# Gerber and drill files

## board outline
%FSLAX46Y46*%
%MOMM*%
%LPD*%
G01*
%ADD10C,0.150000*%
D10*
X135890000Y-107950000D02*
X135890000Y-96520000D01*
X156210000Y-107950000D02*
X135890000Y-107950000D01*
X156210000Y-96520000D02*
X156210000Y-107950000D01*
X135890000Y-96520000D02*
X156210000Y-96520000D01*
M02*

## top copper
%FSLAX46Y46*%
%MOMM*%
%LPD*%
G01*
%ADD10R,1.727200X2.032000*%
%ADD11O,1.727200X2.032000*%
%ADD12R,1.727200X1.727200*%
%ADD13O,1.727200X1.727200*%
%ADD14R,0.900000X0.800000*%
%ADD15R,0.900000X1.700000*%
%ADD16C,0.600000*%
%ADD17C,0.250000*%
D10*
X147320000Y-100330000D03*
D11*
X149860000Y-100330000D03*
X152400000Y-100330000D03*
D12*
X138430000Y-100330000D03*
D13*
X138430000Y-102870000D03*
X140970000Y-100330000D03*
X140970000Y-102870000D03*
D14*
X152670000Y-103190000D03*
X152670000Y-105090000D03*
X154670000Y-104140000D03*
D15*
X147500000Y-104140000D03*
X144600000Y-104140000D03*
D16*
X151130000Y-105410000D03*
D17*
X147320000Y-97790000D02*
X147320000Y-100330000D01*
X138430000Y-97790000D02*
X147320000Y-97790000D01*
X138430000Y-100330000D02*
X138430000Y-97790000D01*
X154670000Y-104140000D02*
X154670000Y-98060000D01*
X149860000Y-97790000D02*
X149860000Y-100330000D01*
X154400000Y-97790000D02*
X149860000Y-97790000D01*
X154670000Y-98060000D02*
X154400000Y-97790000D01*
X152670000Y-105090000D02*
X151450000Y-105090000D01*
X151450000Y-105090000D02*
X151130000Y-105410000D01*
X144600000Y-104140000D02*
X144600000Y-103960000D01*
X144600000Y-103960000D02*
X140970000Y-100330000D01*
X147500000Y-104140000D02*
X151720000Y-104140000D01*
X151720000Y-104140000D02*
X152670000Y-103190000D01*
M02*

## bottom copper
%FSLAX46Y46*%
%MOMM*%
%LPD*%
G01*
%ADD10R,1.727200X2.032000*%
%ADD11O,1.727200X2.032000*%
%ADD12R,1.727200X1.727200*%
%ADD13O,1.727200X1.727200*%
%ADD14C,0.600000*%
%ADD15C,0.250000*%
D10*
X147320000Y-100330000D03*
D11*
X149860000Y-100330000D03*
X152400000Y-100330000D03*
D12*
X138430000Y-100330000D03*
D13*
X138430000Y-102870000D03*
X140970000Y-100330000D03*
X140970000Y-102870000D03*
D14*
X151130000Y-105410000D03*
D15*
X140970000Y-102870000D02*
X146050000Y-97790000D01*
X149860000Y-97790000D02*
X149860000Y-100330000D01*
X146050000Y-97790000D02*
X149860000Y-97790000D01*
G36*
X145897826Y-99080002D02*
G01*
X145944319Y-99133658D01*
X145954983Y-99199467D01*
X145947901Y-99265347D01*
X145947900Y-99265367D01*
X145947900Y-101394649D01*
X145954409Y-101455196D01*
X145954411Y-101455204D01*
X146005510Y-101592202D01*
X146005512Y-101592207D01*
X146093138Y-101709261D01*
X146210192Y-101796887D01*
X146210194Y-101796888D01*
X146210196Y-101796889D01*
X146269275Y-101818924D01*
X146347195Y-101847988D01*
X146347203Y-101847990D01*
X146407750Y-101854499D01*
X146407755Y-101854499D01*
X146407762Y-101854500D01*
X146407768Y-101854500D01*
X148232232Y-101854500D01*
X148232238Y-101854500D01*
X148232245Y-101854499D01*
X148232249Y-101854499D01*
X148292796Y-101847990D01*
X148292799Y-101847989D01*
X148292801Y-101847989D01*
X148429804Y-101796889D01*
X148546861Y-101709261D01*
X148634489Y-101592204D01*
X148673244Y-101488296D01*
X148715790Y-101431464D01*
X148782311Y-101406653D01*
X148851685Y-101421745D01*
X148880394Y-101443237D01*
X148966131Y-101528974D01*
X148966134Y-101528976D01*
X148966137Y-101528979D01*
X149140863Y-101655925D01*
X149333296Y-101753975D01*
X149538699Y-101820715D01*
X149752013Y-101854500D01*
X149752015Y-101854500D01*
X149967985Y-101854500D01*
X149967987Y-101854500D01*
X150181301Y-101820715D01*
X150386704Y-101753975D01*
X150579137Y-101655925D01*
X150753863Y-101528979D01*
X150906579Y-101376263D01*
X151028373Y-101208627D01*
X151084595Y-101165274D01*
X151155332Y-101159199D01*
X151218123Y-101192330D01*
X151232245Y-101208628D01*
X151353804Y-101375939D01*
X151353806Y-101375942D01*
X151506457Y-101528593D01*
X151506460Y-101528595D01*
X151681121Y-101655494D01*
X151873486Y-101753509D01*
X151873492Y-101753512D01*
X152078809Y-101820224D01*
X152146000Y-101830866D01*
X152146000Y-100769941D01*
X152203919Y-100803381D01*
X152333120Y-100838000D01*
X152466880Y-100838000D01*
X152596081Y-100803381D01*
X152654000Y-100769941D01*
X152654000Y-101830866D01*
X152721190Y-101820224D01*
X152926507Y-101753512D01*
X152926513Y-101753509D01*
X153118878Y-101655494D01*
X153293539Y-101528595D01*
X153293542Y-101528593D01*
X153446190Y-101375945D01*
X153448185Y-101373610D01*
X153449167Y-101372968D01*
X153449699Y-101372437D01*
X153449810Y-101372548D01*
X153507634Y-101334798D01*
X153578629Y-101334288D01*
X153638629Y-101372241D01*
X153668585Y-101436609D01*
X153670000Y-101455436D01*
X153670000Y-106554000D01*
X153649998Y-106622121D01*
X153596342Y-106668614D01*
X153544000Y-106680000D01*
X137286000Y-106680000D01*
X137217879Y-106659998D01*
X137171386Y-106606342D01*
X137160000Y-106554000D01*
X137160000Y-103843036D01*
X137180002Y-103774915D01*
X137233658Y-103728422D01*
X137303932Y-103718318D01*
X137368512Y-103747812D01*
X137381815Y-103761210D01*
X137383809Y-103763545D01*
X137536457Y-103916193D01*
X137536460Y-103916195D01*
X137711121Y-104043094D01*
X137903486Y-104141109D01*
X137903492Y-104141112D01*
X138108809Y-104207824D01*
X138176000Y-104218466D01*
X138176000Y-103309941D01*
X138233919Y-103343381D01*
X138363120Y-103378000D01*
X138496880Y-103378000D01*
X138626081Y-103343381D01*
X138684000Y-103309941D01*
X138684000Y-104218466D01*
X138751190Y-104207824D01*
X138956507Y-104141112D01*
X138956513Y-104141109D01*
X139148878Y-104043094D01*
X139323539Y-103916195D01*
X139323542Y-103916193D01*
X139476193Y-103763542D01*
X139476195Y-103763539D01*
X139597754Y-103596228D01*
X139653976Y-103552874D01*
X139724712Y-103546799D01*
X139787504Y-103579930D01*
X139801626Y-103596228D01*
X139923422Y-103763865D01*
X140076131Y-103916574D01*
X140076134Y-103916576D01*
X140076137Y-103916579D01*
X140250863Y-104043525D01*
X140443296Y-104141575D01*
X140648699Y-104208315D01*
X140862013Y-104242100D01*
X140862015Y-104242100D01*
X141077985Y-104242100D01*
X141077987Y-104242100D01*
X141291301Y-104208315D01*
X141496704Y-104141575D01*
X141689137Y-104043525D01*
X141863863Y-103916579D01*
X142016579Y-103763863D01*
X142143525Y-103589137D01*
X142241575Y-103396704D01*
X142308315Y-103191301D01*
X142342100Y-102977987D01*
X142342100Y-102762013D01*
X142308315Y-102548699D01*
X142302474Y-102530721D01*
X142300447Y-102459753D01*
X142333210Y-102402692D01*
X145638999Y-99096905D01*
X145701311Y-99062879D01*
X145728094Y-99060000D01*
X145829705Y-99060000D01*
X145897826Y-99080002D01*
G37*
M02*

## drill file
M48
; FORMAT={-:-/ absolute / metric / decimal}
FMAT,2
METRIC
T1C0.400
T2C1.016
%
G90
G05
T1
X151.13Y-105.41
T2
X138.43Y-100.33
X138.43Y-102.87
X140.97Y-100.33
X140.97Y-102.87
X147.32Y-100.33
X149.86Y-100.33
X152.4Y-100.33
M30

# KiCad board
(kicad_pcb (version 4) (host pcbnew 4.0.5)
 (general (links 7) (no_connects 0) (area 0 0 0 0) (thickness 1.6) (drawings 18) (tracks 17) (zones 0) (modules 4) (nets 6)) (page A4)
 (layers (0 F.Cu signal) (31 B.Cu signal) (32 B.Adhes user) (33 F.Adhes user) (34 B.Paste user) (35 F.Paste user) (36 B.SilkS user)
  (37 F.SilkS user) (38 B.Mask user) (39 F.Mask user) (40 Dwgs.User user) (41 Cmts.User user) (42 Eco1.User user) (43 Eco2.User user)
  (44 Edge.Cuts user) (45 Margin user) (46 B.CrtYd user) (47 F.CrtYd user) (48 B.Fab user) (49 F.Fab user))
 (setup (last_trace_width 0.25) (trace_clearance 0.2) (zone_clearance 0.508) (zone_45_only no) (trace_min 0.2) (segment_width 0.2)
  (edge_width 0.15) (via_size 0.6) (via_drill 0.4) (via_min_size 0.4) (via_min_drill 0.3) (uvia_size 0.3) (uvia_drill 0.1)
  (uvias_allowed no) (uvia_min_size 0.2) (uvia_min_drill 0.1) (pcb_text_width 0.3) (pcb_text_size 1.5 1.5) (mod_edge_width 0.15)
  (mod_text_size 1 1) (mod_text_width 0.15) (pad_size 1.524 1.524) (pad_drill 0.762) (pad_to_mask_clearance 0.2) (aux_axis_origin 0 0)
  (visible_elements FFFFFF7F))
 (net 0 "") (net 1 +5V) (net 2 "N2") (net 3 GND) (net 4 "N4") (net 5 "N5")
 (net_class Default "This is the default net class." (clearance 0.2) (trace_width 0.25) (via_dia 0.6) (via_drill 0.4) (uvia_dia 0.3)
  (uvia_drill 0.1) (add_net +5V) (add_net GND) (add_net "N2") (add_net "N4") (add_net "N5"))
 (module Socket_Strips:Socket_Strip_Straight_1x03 (layer F.Cu) (at 147.32 100.33)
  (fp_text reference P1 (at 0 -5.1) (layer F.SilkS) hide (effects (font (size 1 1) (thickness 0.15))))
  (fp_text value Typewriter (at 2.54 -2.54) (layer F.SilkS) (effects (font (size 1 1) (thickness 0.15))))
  (pad 1 thru_hole rect (at 0 0) (size 1.7272 2.032) (drill 1.016) (layers *.Cu *.Mask) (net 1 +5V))
  (pad 2 thru_hole oval (at 2.54 0) (size 1.7272 2.032) (drill 1.016) (layers *.Cu *.Mask) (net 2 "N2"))
  (pad 3 thru_hole oval (at 5.08 0) (size 1.7272 2.032) (drill 1.016) (layers *.Cu *.Mask) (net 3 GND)))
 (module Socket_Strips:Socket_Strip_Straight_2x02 (layer F.Cu) (at 138.43 100.33)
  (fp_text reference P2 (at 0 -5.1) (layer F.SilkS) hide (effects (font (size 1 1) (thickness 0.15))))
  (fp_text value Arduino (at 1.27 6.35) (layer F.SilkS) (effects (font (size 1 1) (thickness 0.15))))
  (pad 1 thru_hole rect (at 0 0) (size 1.7272 1.7272) (drill 1.016) (layers *.Cu *.Mask) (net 1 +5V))
  (pad 2 thru_hole oval (at 0 2.54) (size 1.7272 1.7272) (drill 1.016) (layers *.Cu *.Mask) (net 3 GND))
  (pad 3 thru_hole oval (at 2.54 0) (size 1.7272 1.7272) (drill 1.016) (layers *.Cu *.Mask) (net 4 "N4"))
  (pad 4 thru_hole oval (at 2.54 2.54) (size 1.7272 1.7272) (drill 1.016) (layers *.Cu *.Mask) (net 2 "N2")))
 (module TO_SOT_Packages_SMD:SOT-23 (layer F.Cu) (at 153.67 104.14)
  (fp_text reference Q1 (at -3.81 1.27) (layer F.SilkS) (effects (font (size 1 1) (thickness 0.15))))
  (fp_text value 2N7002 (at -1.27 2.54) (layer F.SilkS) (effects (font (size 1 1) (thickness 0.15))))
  (pad 1 smd rect (at -1 -0.95) (size 0.9 0.8) (layers F.Cu F.Paste F.Mask) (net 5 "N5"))
  (pad 2 smd rect (at -1 0.95) (size 0.9 0.8) (layers F.Cu F.Paste F.Mask) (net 3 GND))
  (pad 3 smd rect (at 1 0) (size 0.9 0.8) (layers F.Cu F.Paste F.Mask) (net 2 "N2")))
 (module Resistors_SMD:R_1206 (layer F.Cu) (at 146.05 104.14 180)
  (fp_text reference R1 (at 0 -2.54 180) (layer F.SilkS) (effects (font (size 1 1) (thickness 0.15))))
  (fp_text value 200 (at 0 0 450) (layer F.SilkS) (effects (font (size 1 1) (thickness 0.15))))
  (pad 1 smd rect (at -1.45 0 180) (size 0.9 1.7) (layers F.Cu F.Paste F.Mask) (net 5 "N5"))
  (pad 2 smd rect (at 1.45 0 180) (size 0.9 1.7) (layers F.Cu F.Paste F.Mask) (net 4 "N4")))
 (gr_line (start 135.89 107.95) (end 135.89 96.52) (angle 90) (layer Edge.Cuts) (width 0.15))
 (gr_line (start 156.21 107.95) (end 135.89 107.95) (angle 90) (layer Edge.Cuts) (width 0.15))
 (gr_line (start 156.21 96.52) (end 156.21 107.95) (angle 90) (layer Edge.Cuts) (width 0.15))
 (gr_line (start 135.89 96.52) (end 156.21 96.52) (angle 90) (layer Edge.Cuts) (width 0.15))
 (segment (start 147.32 97.79) (end 147.32 100.33) (width 0.25) (layer F.Cu) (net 1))
 (segment (start 138.43 97.79) (end 147.32 97.79) (width 0.25) (layer F.Cu) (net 1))
 (segment (start 138.43 100.33) (end 138.43 97.79) (width 0.25) (layer F.Cu) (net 1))
 (segment (start 154.67 104.14) (end 154.67 98.06) (width 0.25) (layer F.Cu) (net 2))
 (segment (start 149.86 97.79) (end 149.86 100.33) (width 0.25) (layer F.Cu) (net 2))
 (segment (start 154.4 97.79) (end 149.86 97.79) (width 0.25) (layer F.Cu) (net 2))
 (segment (start 154.67 98.06) (end 154.4 97.79) (width 0.25) (layer F.Cu) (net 2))
 (segment (start 140.97 102.87) (end 146.05 97.79) (width 0.25) (layer B.Cu) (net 2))
 (segment (start 149.86 97.79) (end 149.86 100.33) (width 0.25) (layer B.Cu) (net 2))
 (segment (start 146.05 97.79) (end 149.86 97.79) (width 0.25) (layer B.Cu) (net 2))
 (segment (start 152.67 105.09) (end 151.45 105.09) (width 0.25) (layer F.Cu) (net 3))
 (via (at 151.13 105.41) (size 0.6) (drill 0.4) (layers F.Cu B.Cu) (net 3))
 (segment (start 151.45 105.09) (end 151.13 105.41) (width 0.25) (layer F.Cu) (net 3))
 (segment (start 144.6 104.14) (end 144.6 103.96) (width 0.25) (layer F.Cu) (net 4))
 (segment (start 144.6 103.96) (end 140.97 100.33) (width 0.25) (layer F.Cu) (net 4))
 (segment (start 147.5 104.14) (end 151.72 104.14) (width 0.25) (layer F.Cu) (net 5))
 (segment (start 151.72 104.14) (end 152.67 103.19) (width 0.25) (layer F.Cu) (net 5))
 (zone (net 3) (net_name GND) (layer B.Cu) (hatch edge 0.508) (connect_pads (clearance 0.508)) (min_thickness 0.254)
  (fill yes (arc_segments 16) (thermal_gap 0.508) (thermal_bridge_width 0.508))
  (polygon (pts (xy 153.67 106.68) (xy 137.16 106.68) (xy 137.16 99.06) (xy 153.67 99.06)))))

